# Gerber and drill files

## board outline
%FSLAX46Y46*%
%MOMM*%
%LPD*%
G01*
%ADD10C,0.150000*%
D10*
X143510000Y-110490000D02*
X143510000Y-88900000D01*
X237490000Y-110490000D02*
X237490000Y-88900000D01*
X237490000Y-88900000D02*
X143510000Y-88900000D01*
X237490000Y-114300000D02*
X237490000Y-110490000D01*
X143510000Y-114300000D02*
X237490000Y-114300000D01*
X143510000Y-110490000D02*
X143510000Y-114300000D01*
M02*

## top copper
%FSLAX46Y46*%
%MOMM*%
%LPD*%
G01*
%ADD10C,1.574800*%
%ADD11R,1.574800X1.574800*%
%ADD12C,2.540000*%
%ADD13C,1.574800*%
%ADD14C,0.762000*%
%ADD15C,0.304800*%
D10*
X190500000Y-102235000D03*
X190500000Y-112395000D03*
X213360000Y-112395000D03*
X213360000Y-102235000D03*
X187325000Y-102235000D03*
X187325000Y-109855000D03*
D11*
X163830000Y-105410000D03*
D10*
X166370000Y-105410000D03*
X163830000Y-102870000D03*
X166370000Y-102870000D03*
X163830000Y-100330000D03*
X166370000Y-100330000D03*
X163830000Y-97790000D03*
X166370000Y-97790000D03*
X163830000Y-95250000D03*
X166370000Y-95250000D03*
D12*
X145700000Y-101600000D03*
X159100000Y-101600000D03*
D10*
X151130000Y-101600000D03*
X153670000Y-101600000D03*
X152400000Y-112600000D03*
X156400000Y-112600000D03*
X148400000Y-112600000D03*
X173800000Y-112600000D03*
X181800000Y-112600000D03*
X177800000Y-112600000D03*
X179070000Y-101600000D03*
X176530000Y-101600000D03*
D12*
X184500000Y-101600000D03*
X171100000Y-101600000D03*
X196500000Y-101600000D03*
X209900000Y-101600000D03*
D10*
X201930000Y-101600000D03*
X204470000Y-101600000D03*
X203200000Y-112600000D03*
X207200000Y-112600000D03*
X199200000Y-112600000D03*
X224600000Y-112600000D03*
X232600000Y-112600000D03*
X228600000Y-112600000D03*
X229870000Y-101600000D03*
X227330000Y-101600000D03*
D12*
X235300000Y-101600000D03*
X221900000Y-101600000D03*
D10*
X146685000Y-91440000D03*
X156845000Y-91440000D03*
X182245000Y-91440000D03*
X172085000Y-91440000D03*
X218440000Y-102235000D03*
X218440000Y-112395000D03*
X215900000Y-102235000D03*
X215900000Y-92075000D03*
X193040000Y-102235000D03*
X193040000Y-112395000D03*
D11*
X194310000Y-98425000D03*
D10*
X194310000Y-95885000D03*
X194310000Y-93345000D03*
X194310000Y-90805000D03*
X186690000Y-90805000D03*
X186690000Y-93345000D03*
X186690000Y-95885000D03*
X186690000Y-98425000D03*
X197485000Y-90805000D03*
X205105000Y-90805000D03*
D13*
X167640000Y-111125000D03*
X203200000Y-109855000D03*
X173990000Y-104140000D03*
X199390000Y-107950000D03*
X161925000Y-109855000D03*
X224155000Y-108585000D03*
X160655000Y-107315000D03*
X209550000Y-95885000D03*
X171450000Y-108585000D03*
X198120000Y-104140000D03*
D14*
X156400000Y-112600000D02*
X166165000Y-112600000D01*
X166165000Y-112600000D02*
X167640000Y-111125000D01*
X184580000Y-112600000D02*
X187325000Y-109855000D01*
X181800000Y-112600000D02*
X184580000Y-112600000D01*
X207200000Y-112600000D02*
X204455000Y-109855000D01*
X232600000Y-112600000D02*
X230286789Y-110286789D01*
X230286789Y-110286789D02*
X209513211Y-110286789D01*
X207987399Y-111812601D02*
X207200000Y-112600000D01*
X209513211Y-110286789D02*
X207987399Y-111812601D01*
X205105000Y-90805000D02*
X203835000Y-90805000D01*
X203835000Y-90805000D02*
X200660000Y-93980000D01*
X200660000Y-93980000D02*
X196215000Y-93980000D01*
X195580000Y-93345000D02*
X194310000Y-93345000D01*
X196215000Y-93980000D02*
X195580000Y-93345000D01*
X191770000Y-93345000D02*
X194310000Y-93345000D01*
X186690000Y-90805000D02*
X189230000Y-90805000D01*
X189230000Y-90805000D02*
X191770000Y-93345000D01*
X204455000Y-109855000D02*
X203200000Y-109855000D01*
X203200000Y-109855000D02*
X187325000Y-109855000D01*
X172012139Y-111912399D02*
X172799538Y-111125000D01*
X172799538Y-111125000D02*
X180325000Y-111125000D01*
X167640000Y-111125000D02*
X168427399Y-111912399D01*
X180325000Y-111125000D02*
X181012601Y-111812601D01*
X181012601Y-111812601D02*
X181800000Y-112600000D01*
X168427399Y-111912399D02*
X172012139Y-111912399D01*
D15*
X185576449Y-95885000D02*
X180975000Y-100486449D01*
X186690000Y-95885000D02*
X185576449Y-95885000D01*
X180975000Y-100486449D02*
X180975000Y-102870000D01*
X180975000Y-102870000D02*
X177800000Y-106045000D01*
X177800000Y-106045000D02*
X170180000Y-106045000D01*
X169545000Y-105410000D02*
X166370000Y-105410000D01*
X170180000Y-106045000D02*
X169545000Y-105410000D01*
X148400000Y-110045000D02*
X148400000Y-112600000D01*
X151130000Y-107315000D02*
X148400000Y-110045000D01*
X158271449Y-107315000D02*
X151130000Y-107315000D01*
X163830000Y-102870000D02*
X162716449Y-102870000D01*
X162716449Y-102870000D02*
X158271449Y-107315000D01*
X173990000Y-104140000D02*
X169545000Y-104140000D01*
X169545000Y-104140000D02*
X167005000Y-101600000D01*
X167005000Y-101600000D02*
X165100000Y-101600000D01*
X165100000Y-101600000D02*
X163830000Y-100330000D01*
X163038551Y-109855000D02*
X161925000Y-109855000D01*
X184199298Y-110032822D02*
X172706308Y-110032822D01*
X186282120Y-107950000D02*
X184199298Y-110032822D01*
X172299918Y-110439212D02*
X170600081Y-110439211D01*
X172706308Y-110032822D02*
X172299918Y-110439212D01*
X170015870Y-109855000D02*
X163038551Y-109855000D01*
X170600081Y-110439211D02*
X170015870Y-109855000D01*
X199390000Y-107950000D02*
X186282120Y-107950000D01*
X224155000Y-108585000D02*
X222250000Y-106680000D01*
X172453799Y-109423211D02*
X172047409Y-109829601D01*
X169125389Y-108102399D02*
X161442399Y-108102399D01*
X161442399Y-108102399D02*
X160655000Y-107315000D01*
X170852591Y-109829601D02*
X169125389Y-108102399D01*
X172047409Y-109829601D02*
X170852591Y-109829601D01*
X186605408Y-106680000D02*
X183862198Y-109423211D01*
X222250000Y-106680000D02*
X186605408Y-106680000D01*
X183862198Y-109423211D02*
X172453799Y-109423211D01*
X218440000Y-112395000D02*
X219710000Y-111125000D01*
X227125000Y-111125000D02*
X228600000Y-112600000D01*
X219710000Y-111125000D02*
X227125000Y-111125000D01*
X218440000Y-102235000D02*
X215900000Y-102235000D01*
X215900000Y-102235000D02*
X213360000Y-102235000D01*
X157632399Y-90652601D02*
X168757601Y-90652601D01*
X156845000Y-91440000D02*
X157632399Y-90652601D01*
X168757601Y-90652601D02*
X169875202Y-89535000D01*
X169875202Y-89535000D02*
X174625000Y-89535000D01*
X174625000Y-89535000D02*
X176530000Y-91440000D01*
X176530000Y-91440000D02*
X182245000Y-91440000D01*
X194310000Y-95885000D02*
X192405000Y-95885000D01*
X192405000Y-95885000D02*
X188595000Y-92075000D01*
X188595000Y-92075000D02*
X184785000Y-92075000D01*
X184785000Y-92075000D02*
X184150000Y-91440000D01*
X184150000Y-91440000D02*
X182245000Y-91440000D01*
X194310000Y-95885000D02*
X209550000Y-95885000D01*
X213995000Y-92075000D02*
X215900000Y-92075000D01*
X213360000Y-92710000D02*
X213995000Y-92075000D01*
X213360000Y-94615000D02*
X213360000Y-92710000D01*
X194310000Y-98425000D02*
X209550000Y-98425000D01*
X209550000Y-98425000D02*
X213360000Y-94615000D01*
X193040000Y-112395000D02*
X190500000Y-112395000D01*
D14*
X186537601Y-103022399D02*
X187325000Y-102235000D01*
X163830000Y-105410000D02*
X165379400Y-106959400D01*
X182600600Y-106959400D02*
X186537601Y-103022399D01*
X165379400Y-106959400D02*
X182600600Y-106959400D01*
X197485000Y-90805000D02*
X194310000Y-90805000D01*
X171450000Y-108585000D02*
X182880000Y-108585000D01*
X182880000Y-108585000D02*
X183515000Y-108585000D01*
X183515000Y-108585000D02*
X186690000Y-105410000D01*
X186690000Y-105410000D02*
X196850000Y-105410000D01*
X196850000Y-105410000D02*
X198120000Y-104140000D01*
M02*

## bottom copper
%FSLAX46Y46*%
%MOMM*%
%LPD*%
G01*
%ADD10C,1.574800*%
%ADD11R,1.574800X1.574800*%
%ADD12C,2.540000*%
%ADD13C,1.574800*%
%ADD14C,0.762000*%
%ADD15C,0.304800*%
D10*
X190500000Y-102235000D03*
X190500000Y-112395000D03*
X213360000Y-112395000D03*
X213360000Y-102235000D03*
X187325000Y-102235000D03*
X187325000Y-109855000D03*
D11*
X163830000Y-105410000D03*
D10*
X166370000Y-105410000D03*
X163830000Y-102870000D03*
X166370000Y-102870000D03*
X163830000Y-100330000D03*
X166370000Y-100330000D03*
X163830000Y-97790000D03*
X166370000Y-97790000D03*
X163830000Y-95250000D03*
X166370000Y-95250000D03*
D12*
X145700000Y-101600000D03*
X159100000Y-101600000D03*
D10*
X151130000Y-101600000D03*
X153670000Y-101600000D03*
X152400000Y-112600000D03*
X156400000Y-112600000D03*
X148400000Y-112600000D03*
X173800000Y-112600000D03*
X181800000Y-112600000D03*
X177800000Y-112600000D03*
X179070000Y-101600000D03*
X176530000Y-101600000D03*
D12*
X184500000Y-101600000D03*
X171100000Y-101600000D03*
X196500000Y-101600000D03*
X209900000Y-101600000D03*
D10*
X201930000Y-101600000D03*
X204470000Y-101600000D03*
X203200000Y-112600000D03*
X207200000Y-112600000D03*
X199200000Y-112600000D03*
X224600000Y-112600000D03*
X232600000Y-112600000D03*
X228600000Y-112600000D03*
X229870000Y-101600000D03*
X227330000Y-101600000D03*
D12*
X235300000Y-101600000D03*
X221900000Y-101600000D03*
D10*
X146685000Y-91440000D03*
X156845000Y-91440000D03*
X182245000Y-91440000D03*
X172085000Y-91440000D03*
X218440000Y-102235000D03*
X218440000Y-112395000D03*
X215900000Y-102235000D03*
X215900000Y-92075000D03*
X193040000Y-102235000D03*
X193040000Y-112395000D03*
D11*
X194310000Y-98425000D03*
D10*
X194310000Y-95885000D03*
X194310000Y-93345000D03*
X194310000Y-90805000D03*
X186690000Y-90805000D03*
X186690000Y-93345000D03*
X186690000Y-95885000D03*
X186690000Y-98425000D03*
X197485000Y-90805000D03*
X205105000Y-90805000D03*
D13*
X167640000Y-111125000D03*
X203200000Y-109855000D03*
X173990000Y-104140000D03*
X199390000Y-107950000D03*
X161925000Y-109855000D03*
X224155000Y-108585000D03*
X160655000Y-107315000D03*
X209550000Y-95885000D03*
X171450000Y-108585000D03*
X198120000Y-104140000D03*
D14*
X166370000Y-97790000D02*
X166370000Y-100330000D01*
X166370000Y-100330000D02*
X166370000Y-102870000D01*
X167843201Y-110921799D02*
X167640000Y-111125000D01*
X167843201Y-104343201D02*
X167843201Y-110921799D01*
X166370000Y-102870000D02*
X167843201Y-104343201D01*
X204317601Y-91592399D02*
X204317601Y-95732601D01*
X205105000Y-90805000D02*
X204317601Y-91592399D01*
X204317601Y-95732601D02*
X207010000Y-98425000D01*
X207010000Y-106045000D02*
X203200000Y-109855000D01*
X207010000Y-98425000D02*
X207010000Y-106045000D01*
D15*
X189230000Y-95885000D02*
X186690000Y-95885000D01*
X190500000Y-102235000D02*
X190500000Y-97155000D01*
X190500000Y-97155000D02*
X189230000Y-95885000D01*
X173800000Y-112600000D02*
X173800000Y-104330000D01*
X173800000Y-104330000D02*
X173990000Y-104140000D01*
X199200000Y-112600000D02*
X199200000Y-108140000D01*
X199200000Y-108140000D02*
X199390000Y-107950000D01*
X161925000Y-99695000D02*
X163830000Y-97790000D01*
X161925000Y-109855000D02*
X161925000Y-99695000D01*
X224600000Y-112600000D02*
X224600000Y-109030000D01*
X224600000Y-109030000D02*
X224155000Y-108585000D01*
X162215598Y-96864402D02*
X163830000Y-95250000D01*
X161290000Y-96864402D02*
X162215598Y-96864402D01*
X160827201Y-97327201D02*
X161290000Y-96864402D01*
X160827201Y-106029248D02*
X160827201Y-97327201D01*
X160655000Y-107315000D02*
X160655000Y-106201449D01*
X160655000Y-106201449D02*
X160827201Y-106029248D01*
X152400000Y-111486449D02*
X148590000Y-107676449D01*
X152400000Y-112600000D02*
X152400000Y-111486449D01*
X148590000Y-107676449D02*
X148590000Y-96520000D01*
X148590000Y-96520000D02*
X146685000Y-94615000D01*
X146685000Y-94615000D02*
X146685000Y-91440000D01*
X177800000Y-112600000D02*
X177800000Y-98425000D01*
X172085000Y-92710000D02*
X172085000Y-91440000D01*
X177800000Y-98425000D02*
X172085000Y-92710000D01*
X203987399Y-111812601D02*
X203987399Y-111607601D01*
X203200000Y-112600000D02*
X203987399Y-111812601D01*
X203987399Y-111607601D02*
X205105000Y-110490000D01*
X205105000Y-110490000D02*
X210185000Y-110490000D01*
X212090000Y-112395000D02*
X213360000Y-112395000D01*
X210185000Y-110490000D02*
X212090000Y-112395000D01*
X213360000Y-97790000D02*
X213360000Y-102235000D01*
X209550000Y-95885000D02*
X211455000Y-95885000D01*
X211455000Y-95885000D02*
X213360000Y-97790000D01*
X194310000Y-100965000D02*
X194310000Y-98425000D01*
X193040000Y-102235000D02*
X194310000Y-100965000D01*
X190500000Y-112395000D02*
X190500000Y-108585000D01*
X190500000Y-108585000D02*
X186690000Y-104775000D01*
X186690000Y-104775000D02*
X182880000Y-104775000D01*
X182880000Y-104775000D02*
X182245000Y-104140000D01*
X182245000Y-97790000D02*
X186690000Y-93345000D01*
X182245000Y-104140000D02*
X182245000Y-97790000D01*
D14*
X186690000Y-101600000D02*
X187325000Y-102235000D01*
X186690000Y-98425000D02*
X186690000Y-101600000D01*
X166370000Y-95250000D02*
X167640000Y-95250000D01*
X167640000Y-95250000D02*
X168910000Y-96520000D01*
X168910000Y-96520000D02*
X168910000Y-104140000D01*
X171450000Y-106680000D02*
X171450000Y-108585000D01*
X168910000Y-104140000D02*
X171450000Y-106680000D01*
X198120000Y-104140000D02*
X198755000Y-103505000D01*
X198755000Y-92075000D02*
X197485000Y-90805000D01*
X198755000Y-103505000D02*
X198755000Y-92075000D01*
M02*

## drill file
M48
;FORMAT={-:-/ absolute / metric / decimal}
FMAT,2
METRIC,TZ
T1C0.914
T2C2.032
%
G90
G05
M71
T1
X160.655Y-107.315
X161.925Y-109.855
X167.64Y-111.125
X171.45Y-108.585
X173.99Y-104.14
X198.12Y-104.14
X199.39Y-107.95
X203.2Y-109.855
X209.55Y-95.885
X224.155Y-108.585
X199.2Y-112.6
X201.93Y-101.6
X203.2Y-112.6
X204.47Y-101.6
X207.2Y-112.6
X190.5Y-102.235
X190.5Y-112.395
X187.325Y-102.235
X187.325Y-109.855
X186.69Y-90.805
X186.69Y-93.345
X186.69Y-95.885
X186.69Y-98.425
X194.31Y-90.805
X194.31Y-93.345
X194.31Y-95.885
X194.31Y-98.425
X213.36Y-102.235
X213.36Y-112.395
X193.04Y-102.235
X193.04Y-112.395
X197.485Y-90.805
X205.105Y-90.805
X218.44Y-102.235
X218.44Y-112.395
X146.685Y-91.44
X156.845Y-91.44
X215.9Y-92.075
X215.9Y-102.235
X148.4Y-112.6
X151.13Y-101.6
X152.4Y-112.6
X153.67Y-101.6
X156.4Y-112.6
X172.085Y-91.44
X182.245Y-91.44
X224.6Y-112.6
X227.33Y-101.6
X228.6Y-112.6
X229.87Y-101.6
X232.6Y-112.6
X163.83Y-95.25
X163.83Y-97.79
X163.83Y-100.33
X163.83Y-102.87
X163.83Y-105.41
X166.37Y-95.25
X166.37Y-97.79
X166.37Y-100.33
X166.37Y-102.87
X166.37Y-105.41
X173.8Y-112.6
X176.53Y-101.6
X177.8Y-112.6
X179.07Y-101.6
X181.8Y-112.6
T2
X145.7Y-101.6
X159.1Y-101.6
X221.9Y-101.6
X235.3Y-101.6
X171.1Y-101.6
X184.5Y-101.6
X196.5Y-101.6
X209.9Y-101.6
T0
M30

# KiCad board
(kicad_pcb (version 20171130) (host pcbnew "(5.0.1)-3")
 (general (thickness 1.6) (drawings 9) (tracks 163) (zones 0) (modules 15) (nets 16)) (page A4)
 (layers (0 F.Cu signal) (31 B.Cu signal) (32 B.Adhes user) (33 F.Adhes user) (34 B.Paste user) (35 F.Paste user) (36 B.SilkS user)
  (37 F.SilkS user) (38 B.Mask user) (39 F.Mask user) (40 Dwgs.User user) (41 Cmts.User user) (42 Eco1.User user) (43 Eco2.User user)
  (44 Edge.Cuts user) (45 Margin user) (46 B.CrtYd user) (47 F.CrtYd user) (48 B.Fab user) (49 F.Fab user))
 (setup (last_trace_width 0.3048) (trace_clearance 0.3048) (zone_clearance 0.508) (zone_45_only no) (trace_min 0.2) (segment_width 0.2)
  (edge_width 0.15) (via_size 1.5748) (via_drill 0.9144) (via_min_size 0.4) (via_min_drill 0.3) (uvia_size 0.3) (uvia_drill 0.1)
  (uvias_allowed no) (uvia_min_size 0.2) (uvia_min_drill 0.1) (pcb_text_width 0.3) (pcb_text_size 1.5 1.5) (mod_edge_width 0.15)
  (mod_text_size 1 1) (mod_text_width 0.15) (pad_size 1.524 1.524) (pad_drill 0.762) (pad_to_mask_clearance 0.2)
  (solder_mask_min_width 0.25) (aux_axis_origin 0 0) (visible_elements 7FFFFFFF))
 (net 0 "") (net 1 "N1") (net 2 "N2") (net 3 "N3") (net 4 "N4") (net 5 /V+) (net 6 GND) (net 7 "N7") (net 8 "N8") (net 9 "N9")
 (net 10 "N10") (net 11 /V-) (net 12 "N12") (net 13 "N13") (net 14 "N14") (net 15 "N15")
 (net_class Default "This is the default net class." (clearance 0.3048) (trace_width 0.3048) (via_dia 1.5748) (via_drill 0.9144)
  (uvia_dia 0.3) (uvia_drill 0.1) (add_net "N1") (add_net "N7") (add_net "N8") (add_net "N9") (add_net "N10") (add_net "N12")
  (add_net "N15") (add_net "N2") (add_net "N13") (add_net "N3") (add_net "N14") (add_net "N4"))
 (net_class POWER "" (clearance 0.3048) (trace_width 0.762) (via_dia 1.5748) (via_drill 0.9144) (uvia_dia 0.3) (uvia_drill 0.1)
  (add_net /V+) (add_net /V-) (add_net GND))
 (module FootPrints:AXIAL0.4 (layer F.Cu) (at 190.5 107.315 90)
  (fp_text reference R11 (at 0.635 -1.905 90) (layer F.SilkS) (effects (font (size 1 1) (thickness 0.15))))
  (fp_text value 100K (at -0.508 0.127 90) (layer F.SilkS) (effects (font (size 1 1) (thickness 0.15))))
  (pad 2 thru_hole circle (at 5.08 0 90) (size 1.5748 1.5748) (drill 0.9144) (layers *.Cu *.Mask F.SilkS) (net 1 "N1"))
  (pad 1 thru_hole circle (at -5.08 0 90) (size 1.5748 1.5748) (drill 0.9144) (layers *.Cu *.Mask F.SilkS) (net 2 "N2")))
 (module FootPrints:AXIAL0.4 (layer F.Cu) (at 213.36 107.315 90)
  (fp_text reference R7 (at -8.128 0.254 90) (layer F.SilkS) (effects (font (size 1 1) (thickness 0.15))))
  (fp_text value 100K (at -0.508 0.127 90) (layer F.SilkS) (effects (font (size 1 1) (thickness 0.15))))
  (pad 1 thru_hole circle (at -5.08 0 90) (size 1.5748 1.5748) (drill 0.9144) (layers *.Cu *.Mask F.SilkS) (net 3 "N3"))
  (pad 2 thru_hole circle (at 5.08 0 90) (size 1.5748 1.5748) (drill 0.9144) (layers *.Cu *.Mask F.SilkS) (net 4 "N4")))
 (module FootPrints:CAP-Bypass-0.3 (layer F.Cu) (at 187.325 106.045 270)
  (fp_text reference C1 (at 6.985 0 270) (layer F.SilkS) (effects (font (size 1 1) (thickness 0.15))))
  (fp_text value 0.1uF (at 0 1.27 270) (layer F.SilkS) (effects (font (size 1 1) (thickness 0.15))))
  (pad 1 thru_hole circle (at -3.81 0 270) (size 1.5748 1.5748) (drill 0.9144) (layers *.Cu *.Mask F.SilkS) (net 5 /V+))
  (pad 2 thru_hole circle (at 3.81 0 270) (size 1.5748 1.5748) (drill 0.9144) (layers *.Cu *.Mask F.SilkS) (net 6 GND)))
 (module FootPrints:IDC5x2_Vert (layer B.Cu) (at 165.1 100.33 270)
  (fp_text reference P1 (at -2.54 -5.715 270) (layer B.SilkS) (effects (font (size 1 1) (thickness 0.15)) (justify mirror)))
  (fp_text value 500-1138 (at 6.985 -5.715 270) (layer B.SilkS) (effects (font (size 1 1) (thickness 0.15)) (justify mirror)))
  (pad 1 thru_hole rect (at 5.08 1.27 270) (size 1.5748 1.5748) (drill 0.9144) (layers *.Cu *.Mask B.SilkS) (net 5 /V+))
  (pad 2 thru_hole circle (at 5.08 -1.27 270) (size 1.5748 1.5748) (drill 0.9144) (layers *.Cu *.Mask B.SilkS) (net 1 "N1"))
  (pad 3 thru_hole circle (at 2.54 1.27 270) (size 1.5748 1.5748) (drill 0.9144) (layers *.Cu *.Mask B.SilkS) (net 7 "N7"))
  (pad 4 thru_hole circle (at 2.54 -1.27 270) (size 1.5748 1.5748) (drill 0.9144) (layers *.Cu *.Mask B.SilkS) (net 6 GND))
  (pad 5 thru_hole circle (at 0 1.27 270) (size 1.5748 1.5748) (drill 0.9144) (layers *.Cu *.Mask B.SilkS) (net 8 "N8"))
  (pad 6 thru_hole circle (at 0 -1.27 270) (size 1.5748 1.5748) (drill 0.9144) (layers *.Cu *.Mask B.SilkS) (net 6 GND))
  (pad 7 thru_hole circle (at -2.54 1.27 270) (size 1.5748 1.5748) (drill 0.9144) (layers *.Cu *.Mask B.SilkS) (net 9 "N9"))
  (pad 8 thru_hole circle (at -2.54 -1.27 270) (size 1.5748 1.5748) (drill 0.9144) (layers *.Cu *.Mask B.SilkS) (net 6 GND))
  (pad 9 thru_hole circle (at -5.08 1.27 270) (size 1.5748 1.5748) (drill 0.9144) (layers *.Cu *.Mask B.SilkS) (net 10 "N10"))
  (pad 10 thru_hole circle (at -5.08 -1.27 270) (size 1.5748 1.5748) (drill 0.9144) (layers *.Cu *.Mask B.SilkS) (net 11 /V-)))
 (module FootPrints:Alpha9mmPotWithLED (layer F.Cu) (at 152.4 101.6)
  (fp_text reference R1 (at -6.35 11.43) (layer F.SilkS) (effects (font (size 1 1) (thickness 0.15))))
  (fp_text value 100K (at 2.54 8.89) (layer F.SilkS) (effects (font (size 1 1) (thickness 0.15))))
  (pad "" thru_hole circle (at -6.7 0) (size 2.54 2.54) (drill 2.032) (layers *.Cu *.Mask F.SilkS))
  (pad "" thru_hole circle (at 6.7 0) (size 2.54 2.54) (drill 2.032) (layers *.Cu *.Mask F.SilkS))
  (pad 4 thru_hole circle (at -1.27 0) (size 1.5748 1.5748) (drill 0.9144) (layers *.Cu *.Mask F.SilkS))
  (pad 5 thru_hole circle (at 1.27 0) (size 1.5748 1.5748) (drill 0.9144) (layers *.Cu *.Mask F.SilkS))
  (pad 2 thru_hole circle (at 0 11) (size 1.5748 1.5748) (drill 0.9144) (layers *.Cu *.Mask F.SilkS) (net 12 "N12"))
  (pad 3 thru_hole circle (at 4 11) (size 1.5748 1.5748) (drill 0.9144) (layers *.Cu *.Mask F.SilkS) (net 6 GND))
  (pad 1 thru_hole circle (at -4 11) (size 1.5748 1.5748) (drill 0.9144) (layers *.Cu *.Mask F.SilkS) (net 7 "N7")))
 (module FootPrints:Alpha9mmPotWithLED (layer F.Cu) (at 177.8 101.6)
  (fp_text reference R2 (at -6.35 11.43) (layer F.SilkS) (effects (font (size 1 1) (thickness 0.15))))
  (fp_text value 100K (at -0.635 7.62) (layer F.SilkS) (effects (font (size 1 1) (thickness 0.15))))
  (pad 1 thru_hole circle (at -4 11) (size 1.5748 1.5748) (drill 0.9144) (layers *.Cu *.Mask F.SilkS) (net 8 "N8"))
  (pad 3 thru_hole circle (at 4 11) (size 1.5748 1.5748) (drill 0.9144) (layers *.Cu *.Mask F.SilkS) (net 6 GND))
  (pad 2 thru_hole circle (at 0 11) (size 1.5748 1.5748) (drill 0.9144) (layers *.Cu *.Mask F.SilkS) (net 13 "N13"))
  (pad 5 thru_hole circle (at 1.27 0) (size 1.5748 1.5748) (drill 0.9144) (layers *.Cu *.Mask F.SilkS))
  (pad 4 thru_hole circle (at -1.27 0) (size 1.5748 1.5748) (drill 0.9144) (layers *.Cu *.Mask F.SilkS))
  (pad "" thru_hole circle (at 6.7 0) (size 2.54 2.54) (drill 2.032) (layers *.Cu *.Mask F.SilkS))
  (pad "" thru_hole circle (at -6.7 0) (size 2.54 2.54) (drill 2.032) (layers *.Cu *.Mask F.SilkS)))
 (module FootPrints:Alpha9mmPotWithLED (layer F.Cu) (at 203.2 101.6)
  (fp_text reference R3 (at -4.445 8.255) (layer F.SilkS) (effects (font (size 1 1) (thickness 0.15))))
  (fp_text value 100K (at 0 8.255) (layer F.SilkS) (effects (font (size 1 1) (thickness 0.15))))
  (pad "" thru_hole circle (at -6.7 0) (size 2.54 2.54) (drill 2.032) (layers *.Cu *.Mask F.SilkS))
  (pad "" thru_hole circle (at 6.7 0) (size 2.54 2.54) (drill 2.032) (layers *.Cu *.Mask F.SilkS))
  (pad 4 thru_hole circle (at -1.27 0) (size 1.5748 1.5748) (drill 0.9144) (layers *.Cu *.Mask F.SilkS))
  (pad 5 thru_hole circle (at 1.27 0) (size 1.5748 1.5748) (drill 0.9144) (layers *.Cu *.Mask F.SilkS))
  (pad 2 thru_hole circle (at 0 11) (size 1.5748 1.5748) (drill 0.9144) (layers *.Cu *.Mask F.SilkS) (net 3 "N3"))
  (pad 3 thru_hole circle (at 4 11) (size 1.5748 1.5748) (drill 0.9144) (layers *.Cu *.Mask F.SilkS) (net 6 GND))
  (pad 1 thru_hole circle (at -4 11) (size 1.5748 1.5748) (drill 0.9144) (layers *.Cu *.Mask F.SilkS) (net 9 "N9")))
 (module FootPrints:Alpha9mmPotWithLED (layer F.Cu) (at 228.6 101.6)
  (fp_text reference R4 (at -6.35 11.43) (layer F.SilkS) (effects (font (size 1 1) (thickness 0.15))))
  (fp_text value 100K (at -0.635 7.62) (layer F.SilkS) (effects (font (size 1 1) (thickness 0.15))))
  (pad 1 thru_hole circle (at -4 11) (size 1.5748 1.5748) (drill 0.9144) (layers *.Cu *.Mask F.SilkS) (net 10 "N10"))
  (pad 3 thru_hole circle (at 4 11) (size 1.5748 1.5748) (drill 0.9144) (layers *.Cu *.Mask F.SilkS) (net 6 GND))
  (pad 2 thru_hole circle (at 0 11) (size 1.5748 1.5748) (drill 0.9144) (layers *.Cu *.Mask F.SilkS) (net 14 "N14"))
  (pad 5 thru_hole circle (at 1.27 0) (size 1.5748 1.5748) (drill 0.9144) (layers *.Cu *.Mask F.SilkS))
  (pad 4 thru_hole circle (at -1.27 0) (size 1.5748 1.5748) (drill 0.9144) (layers *.Cu *.Mask F.SilkS))
  (pad "" thru_hole circle (at 6.7 0) (size 2.54 2.54) (drill 2.032) (layers *.Cu *.Mask F.SilkS))
  (pad "" thru_hole circle (at -6.7 0) (size 2.54 2.54) (drill 2.032) (layers *.Cu *.Mask F.SilkS)))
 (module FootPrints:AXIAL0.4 (layer F.Cu) (at 151.765 91.44)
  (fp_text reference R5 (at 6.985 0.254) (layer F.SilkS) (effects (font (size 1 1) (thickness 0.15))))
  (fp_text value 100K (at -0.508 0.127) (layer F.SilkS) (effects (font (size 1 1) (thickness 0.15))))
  (pad 1 thru_hole circle (at -5.08 0) (size 1.5748 1.5748) (drill 0.9144) (layers *.Cu *.Mask F.SilkS) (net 12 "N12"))
  (pad 2 thru_hole circle (at 5.08 0) (size 1.5748 1.5748) (drill 0.9144) (layers *.Cu *.Mask F.SilkS) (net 4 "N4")))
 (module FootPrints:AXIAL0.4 (layer F.Cu) (at 177.165 91.44)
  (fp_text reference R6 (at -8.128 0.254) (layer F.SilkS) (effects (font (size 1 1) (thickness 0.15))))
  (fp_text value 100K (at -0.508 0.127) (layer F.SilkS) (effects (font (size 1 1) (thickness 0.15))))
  (pad 2 thru_hole circle (at 5.08 0) (size 1.5748 1.5748) (drill 0.9144) (layers *.Cu *.Mask F.SilkS) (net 4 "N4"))
  (pad 1 thru_hole circle (at -5.08 0) (size 1.5748 1.5748) (drill 0.9144) (layers *.Cu *.Mask F.SilkS) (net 13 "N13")))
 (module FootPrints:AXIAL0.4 (layer F.Cu) (at 218.44 107.315 90)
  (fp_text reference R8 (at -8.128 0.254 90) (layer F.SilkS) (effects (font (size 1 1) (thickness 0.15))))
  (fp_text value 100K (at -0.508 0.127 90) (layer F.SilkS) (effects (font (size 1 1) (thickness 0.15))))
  (pad 2 thru_hole circle (at 5.08 0 90) (size 1.5748 1.5748) (drill 0.9144) (layers *.Cu *.Mask F.SilkS) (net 4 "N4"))
  (pad 1 thru_hole circle (at -5.08 0 90) (size 1.5748 1.5748) (drill 0.9144) (layers *.Cu *.Mask F.SilkS) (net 14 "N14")))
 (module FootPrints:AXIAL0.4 (layer F.Cu) (at 215.9 97.155 90)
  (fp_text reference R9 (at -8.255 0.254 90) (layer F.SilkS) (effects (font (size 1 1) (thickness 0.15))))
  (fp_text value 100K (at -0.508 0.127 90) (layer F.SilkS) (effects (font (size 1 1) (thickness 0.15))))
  (pad 1 thru_hole circle (at -5.08 0 90) (size 1.5748 1.5748) (drill 0.9144) (layers *.Cu *.Mask F.SilkS) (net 4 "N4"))
  (pad 2 thru_hole circle (at 5.08 0 90) (size 1.5748 1.5748) (drill 0.9144) (layers *.Cu *.Mask F.SilkS) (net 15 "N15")))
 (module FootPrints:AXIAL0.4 (layer F.Cu) (at 193.04 107.315 270)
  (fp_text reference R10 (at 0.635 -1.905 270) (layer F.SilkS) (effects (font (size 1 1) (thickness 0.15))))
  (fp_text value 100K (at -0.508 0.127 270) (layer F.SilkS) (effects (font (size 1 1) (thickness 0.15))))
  (pad 1 thru_hole circle (at -5.08 0 270) (size 1.5748 1.5748) (drill 0.9144) (layers *.Cu *.Mask F.SilkS) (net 15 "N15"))
  (pad 2 thru_hole circle (at 5.08 0 270) (size 1.5748 1.5748) (drill 0.9144) (layers *.Cu *.Mask F.SilkS) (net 2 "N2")))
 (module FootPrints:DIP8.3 (layer F.Cu) (at 190.5 94.615 90)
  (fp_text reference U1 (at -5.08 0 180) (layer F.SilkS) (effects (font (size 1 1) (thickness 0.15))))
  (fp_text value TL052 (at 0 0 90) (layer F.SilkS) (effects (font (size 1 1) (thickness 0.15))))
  (pad 1 thru_hole rect (at -3.81 3.81 90) (size 1.5748 1.5748) (drill 0.9144) (layers *.Cu *.Mask F.SilkS) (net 15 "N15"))
  (pad 2 thru_hole circle (at -1.27 3.81 90) (size 1.5748 1.5748) (drill 0.9144) (layers *.Cu *.Mask F.SilkS) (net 4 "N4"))
  (pad 3 thru_hole circle (at 1.27 3.81 90) (size 1.5748 1.5748) (drill 0.9144) (layers *.Cu *.Mask F.SilkS) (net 6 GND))
  (pad 4 thru_hole circle (at 3.81 3.81 90) (size 1.5748 1.5748) (drill 0.9144) (layers *.Cu *.Mask F.SilkS) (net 11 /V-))
  (pad 5 thru_hole circle (at 3.81 -3.81 90) (size 1.5748 1.5748) (drill 0.9144) (layers *.Cu *.Mask F.SilkS) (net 6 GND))
  (pad 6 thru_hole circle (at 1.27 -3.81 90) (size 1.5748 1.5748) (drill 0.9144) (layers *.Cu *.Mask F.SilkS) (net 2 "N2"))
  (pad 7 thru_hole circle (at -1.27 -3.81 90) (size 1.5748 1.5748) (drill 0.9144) (layers *.Cu *.Mask F.SilkS) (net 1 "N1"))
  (pad 8 thru_hole circle (at -3.81 -3.81 90) (size 1.5748 1.5748) (drill 0.9144) (layers *.Cu *.Mask F.SilkS) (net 5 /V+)))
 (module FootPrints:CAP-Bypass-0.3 (layer F.Cu) (at 201.295 90.805)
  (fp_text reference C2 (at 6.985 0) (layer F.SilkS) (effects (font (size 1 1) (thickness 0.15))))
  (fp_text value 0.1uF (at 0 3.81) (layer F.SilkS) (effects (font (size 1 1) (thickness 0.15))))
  (pad 1 thru_hole circle (at -3.81 0) (size 1.5748 1.5748) (drill 0.9144) (layers *.Cu *.Mask F.SilkS) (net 11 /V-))
  (pad 2 thru_hole circle (at 3.81 0) (size 1.5748 1.5748) (drill 0.9144) (layers *.Cu *.Mask F.SilkS) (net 6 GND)))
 (gr_line (start 143.51 110.49) (end 143.51 88.9) (layer Edge.Cuts) (width 0.15))
 (gr_line (start 237.49 110.49) (end 237.49 88.9) (layer Edge.Cuts) (width 0.15))
 (gr_line (start 237.49 88.9) (end 143.51 88.9) (layer Edge.Cuts) (width 0.15))
 (gr_line (start 237.49 114.3) (end 237.49 110.49) (layer Edge.Cuts) (width 0.15))
 (gr_line (start 143.51 114.3) (end 237.49 114.3) (layer Edge.Cuts) (width 0.15))
 (gr_line (start 143.51 110.49) (end 143.51 114.3) (layer Edge.Cuts) (width 0.15))
 (segment (start 156.4 112.6) (end 166.165 112.6) (width 0.762) (layer F.Cu) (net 6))
 (segment (start 166.165 112.6) (end 167.64 111.125) (width 0.762) (layer F.Cu) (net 6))
 (segment (start 184.58 112.6) (end 187.325 109.855) (width 0.762) (layer F.Cu) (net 6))
 (segment (start 181.8 112.6) (end 184.58 112.6) (width 0.762) (layer F.Cu) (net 6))
 (segment (start 207.2 112.6) (end 204.455 109.855) (width 0.762) (layer F.Cu) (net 6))
 (segment (start 232.6 112.6) (end 230.286789 110.286789) (width 0.762) (layer F.Cu) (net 6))
 (segment (start 230.286789 110.286789) (end 209.513211 110.286789) (width 0.762) (layer F.Cu) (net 6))
 (segment (start 207.987399 111.812601) (end 207.2 112.6) (width 0.762) (layer F.Cu) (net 6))
 (segment (start 209.513211 110.286789) (end 207.987399 111.812601) (width 0.762) (layer F.Cu) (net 6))
 (segment (start 166.37 97.79) (end 166.37 100.33) (width 0.762) (layer B.Cu) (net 6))
 (segment (start 166.37 100.33) (end 166.37 102.87) (width 0.762) (layer B.Cu) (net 6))
 (via (at 167.64 111.125) (size 1.5748) (drill 0.9144) (layers F.Cu B.Cu) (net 6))
 (segment (start 167.843201 110.921799) (end 167.64 111.125) (width 0.762) (layer B.Cu) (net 6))
 (segment (start 167.843201 104.343201) (end 167.843201 110.921799) (width 0.762) (layer B.Cu) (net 6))
 (segment (start 166.37 102.87) (end 167.843201 104.343201) (width 0.762) (layer B.Cu) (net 6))
 (segment (start 205.105 90.805) (end 203.835 90.805) (width 0.762) (layer F.Cu) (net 6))
 (segment (start 203.835 90.805) (end 200.66 93.98) (width 0.762) (layer F.Cu) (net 6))
 (segment (start 200.66 93.98) (end 196.215 93.98) (width 0.762) (layer F.Cu) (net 6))
 (segment (start 195.58 93.345) (end 194.31 93.345) (width 0.762) (layer F.Cu) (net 6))
 (segment (start 196.215 93.98) (end 195.58 93.345) (width 0.762) (layer F.Cu) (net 6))
 (segment (start 191.77 93.345) (end 194.31 93.345) (width 0.762) (layer F.Cu) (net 6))
 (segment (start 186.69 90.805) (end 189.23 90.805) (width 0.762) (layer F.Cu) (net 6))
 (segment (start 189.23 90.805) (end 191.77 93.345) (width 0.762) (layer F.Cu) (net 6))
 (segment (start 204.317601 91.592399) (end 204.317601 95.732601) (width 0.762) (layer B.Cu) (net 6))
 (segment (start 205.105 90.805) (end 204.317601 91.592399) (width 0.762) (layer B.Cu) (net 6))
 (segment (start 204.317601 95.732601) (end 207.01 98.425) (width 0.762) (layer B.Cu) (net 6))
 (via (at 203.2 109.855) (size 1.5748) (drill 0.9144) (layers F.Cu B.Cu) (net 6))
 (segment (start 207.01 106.045) (end 203.2 109.855) (width 0.762) (layer B.Cu) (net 6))
 (segment (start 207.01 98.425) (end 207.01 106.045) (width 0.762) (layer B.Cu) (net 6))
 (segment (start 204.455 109.855) (end 203.2 109.855) (width 0.762) (layer F.Cu) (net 6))
 (segment (start 203.2 109.855) (end 187.325 109.855) (width 0.762) (layer F.Cu) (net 6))
 (segment (start 172.012139 111.912399) (end 172.799538 111.125) (width 0.762) (layer F.Cu) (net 6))
 (segment (start 172.799538 111.125) (end 180.325 111.125) (width 0.762) (layer F.Cu) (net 6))
 (segment (start 167.64 111.125) (end 168.427399 111.912399) (width 0.762) (layer F.Cu) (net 6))
 (segment (start 180.325 111.125) (end 181.012601 111.812601) (width 0.762) (layer F.Cu) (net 6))
 (segment (start 181.012601 111.812601) (end 181.8 112.6) (width 0.762) (layer F.Cu) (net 6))
 (segment (start 168.427399 111.912399) (end 172.012139 111.912399) (width 0.762) (layer F.Cu) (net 6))
 (segment (start 189.23 95.885) (end 186.69 95.885) (width 0.3048) (layer B.Cu) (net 1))
 (segment (start 190.5 102.235) (end 190.5 97.155) (width 0.3048) (layer B.Cu) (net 1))
 (segment (start 190.5 97.155) (end 189.23 95.885) (width 0.3048) (layer B.Cu) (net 1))
 (segment (start 185.576449 95.885) (end 180.975 100.486449) (width 0.3048) (layer F.Cu) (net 1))
 (segment (start 186.69 95.885) (end 185.576449 95.885) (width 0.3048) (layer F.Cu) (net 1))
 (segment (start 180.975 100.486449) (end 180.975 102.87) (width 0.3048) (layer F.Cu) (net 1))
 (segment (start 180.975 102.87) (end 177.8 106.045) (width 0.3048) (layer F.Cu) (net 1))
 (segment (start 177.8 106.045) (end 170.18 106.045) (width 0.3048) (layer F.Cu) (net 1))
 (segment (start 169.545 105.41) (end 166.37 105.41) (width 0.3048) (layer F.Cu) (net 1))
 (segment (start 170.18 106.045) (end 169.545 105.41) (width 0.3048) (layer F.Cu) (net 1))
 (segment (start 148.4 110.045) (end 148.4 112.6) (width 0.3048) (layer F.Cu) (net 7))
 (segment (start 151.13 107.315) (end 148.4 110.045) (width 0.3048) (layer F.Cu) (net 7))
 (segment (start 158.271449 107.315) (end 151.13 107.315) (width 0.3048) (layer F.Cu) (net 7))
 (segment (start 163.83 102.87) (end 162.716449 102.87) (width 0.3048) (layer F.Cu) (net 7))
 (segment (start 162.716449 102.87) (end 158.271449 107.315) (width 0.3048) (layer F.Cu) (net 7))
 (via (at 173.99 104.14) (size 1.5748) (drill 0.9144) (layers F.Cu B.Cu) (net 8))
 (segment (start 173.8 112.6) (end 173.8 104.33) (width 0.3048) (layer B.Cu) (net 8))
 (segment (start 173.8 104.33) (end 173.99 104.14) (width 0.3048) (layer B.Cu) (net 8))
 (segment (start 173.99 104.14) (end 169.545 104.14) (width 0.3048) (layer F.Cu) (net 8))
 (segment (start 169.545 104.14) (end 167.005 101.6) (width 0.3048) (layer F.Cu) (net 8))
 (segment (start 167.005 101.6) (end 165.1 101.6) (width 0.3048) (layer F.Cu) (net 8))
 (segment (start 165.1 101.6) (end 163.83 100.33) (width 0.3048) (layer F.Cu) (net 8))
 (via (at 199.39 107.95) (size 1.5748) (drill 0.9144) (layers F.Cu B.Cu) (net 9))
 (segment (start 199.2 112.6) (end 199.2 108.14) (width 0.3048) (layer B.Cu) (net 9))
 (segment (start 199.2 108.14) (end 199.39 107.95) (width 0.3048) (layer B.Cu) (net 9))
 (via (at 161.925 109.855) (size 1.5748) (drill 0.9144) (layers F.Cu B.Cu) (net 9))
 (segment (start 161.925 99.695) (end 163.83 97.79) (width 0.3048) (layer B.Cu) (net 9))
 (segment (start 161.925 109.855) (end 161.925 99.695) (width 0.3048) (layer B.Cu) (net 9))
 (segment (start 163.038551 109.855) (end 161.925 109.855) (width 0.3048) (layer F.Cu) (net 9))
 (segment (start 184.199298 110.032822) (end 172.706308 110.032822) (width 0.3048) (layer F.Cu) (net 9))
 (segment (start 186.28212 107.95) (end 184.199298 110.032822) (width 0.3048) (layer F.Cu) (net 9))
 (segment (start 172.299918 110.439212) (end 170.600081 110.439211) (width 0.3048) (layer F.Cu) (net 9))
 (segment (start 172.706308 110.032822) (end 172.299918 110.439212) (width 0.3048) (layer F.Cu) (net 9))
 (segment (start 170.01587 109.855) (end 163.038551 109.855) (width 0.3048) (layer F.Cu) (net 9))
 (segment (start 170.600081 110.439211) (end 170.01587 109.855) (width 0.3048) (layer F.Cu) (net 9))
 (segment (start 199.39 107.95) (end 186.28212 107.95) (width 0.3048) (layer F.Cu) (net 9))
 (via (at 224.155 108.585) (size 1.5748) (drill 0.9144) (layers F.Cu B.Cu) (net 10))
 (segment (start 224.6 112.6) (end 224.6 109.03) (width 0.3048) (layer B.Cu) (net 10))
 (segment (start 224.6 109.03) (end 224.155 108.585) (width 0.3048) (layer B.Cu) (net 10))
 (via (at 160.655 107.315) (size 1.5748) (drill 0.9144) (layers F.Cu B.Cu) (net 10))
 (segment (start 162.215598 96.864402) (end 163.83 95.25) (width 0.3048) (layer B.Cu) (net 10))
 (segment (start 161.29 96.864402) (end 162.215598 96.864402) (width 0.3048) (layer B.Cu) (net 10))
 (segment (start 160.827201 97.327201) (end 161.29 96.864402) (width 0.3048) (layer B.Cu) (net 10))
 (segment (start 160.827201 106.029248) (end 160.827201 97.327201) (width 0.3048) (layer B.Cu) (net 10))
 (segment (start 160.655 107.315) (end 160.655 106.201449) (width 0.3048) (layer B.Cu) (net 10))
 (segment (start 160.655 106.201449) (end 160.827201 106.029248) (width 0.3048) (layer B.Cu) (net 10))
 (segment (start 224.155 108.585) (end 222.25 106.68) (width 0.3048) (layer F.Cu) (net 10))
 (segment (start 172.453799 109.423211) (end 172.047409 109.829601) (width 0.3048) (layer F.Cu) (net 10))
 (segment (start 169.125389 108.102399) (end 161.442399 108.102399) (width 0.3048) (layer F.Cu) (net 10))
 (segment (start 161.442399 108.102399) (end 160.655 107.315) (width 0.3048) (layer F.Cu) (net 10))
 (segment (start 170.852591 109.829601) (end 169.125389 108.102399) (width 0.3048) (layer F.Cu) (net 10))
 (segment (start 172.047409 109.829601) (end 170.852591 109.829601) (width 0.3048) (layer F.Cu) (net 10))
 (segment (start 186.605408 106.68) (end 183.862198 109.423211) (width 0.3048) (layer F.Cu) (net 10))
 (segment (start 222.25 106.68) (end 186.605408 106.68) (width 0.3048) (layer F.Cu) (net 10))
 (segment (start 183.862198 109.423211) (end 172.453799 109.423211) (width 0.3048) (layer F.Cu) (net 10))
 (segment (start 152.4 111.486449) (end 148.59 107.676449) (width 0.3048) (layer B.Cu) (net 12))
 (segment (start 152.4 112.6) (end 152.4 111.486449) (width 0.3048) (layer B.Cu) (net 12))
 (segment (start 148.59 107.676449) (end 148.59 96.52) (width 0.3048) (layer B.Cu) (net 12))
 (segment (start 148.59 96.52) (end 146.685 94.615) (width 0.3048) (layer B.Cu) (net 12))
 (segment (start 146.685 94.615) (end 146.685 91.44) (width 0.3048) (layer B.Cu) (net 12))
 (segment (start 177.8 112.6) (end 177.8 98.425) (width 0.3048) (layer B.Cu) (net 13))
 (segment (start 172.085 92.71) (end 172.085 91.44) (width 0.3048) (layer B.Cu) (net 13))
 (segment (start 177.8 98.425) (end 172.085 92.71) (width 0.3048) (layer B.Cu) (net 13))
 (segment (start 203.987399 111.812601) (end 203.987399 111.607601) (width 0.3048) (layer B.Cu) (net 3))
 (segment (start 203.2 112.6) (end 203.987399 111.812601) (width 0.3048) (layer B.Cu) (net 3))
 (segment (start 203.987399 111.607601) (end 205.105 110.49) (width 0.3048) (layer B.Cu) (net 3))
 (segment (start 205.105 110.49) (end 210.185 110.49) (width 0.3048) (layer B.Cu) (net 3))
 (segment (start 212.09 112.395) (end 213.36 112.395) (width 0.3048) (layer B.Cu) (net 3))
 (segment (start 210.185 110.49) (end 212.09 112.395) (width 0.3048) (layer B.Cu) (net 3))
 (segment (start 218.44 112.395) (end 219.71 111.125) (width 0.3048) (layer F.Cu) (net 14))
 (segment (start 227.125 111.125) (end 228.6 112.6) (width 0.3048) (layer F.Cu) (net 14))
 (segment (start 219.71 111.125) (end 227.125 111.125) (width 0.3048) (layer F.Cu) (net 14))
 (segment (start 218.44 102.235) (end 215.9 102.235) (width 0.3048) (layer F.Cu) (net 4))
 (segment (start 215.9 102.235) (end 213.36 102.235) (width 0.3048) (layer F.Cu) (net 4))
 (segment (start 157.632399 90.652601) (end 168.757601 90.652601) (width 0.3048) (layer F.Cu) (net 4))
 (segment (start 156.845 91.44) (end 157.632399 90.652601) (width 0.3048) (layer F.Cu) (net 4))
 (segment (start 168.757601 90.652601) (end 169.875202 89.535) (width 0.3048) (layer F.Cu) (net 4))
 (segment (start 169.875202 89.535) (end 174.625 89.535) (width 0.3048) (layer F.Cu) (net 4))
 (segment (start 174.625 89.535) (end 176.53 91.44) (width 0.3048) (layer F.Cu) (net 4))
 (segment (start 176.53 91.44) (end 182.245 91.44) (width 0.3048) (layer F.Cu) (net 4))
 (segment (start 194.31 95.885) (end 192.405 95.885) (width 0.3048) (layer F.Cu) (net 4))
 (segment (start 192.405 95.885) (end 188.595 92.075) (width 0.3048) (layer F.Cu) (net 4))
 (segment (start 188.595 92.075) (end 184.785 92.075) (width 0.3048) (layer F.Cu) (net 4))
 (segment (start 184.785 92.075) (end 184.15 91.44) (width 0.3048) (layer F.Cu) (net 4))
 (segment (start 184.15 91.44) (end 182.245 91.44) (width 0.3048) (layer F.Cu) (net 4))
 (via (at 209.55 95.885) (size 1.5748) (drill 0.9144) (layers F.Cu B.Cu) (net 4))
 (segment (start 194.31 95.885) (end 209.55 95.885) (width 0.3048) (layer F.Cu) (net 4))
 (segment (start 213.36 97.79) (end 213.36 102.235) (width 0.3048) (layer B.Cu) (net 4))
 (segment (start 209.55 95.885) (end 211.455 95.885) (width 0.3048) (layer B.Cu) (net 4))
 (segment (start 211.455 95.885) (end 213.36 97.79) (width 0.3048) (layer B.Cu) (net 4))
 (segment (start 194.31 100.965) (end 194.31 98.425) (width 0.3048) (layer B.Cu) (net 15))
 (segment (start 193.04 102.235) (end 194.31 100.965) (width 0.3048) (layer B.Cu) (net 15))
 (segment (start 213.995 92.075) (end 215.9 92.075) (width 0.3048) (layer F.Cu) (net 15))
 (segment (start 213.36 92.71) (end 213.995 92.075) (width 0.3048) (layer F.Cu) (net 15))
 (segment (start 213.36 94.615) (end 213.36 92.71) (width 0.3048) (layer F.Cu) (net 15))
 (segment (start 194.31 98.425) (end 209.55 98.425) (width 0.3048) (layer F.Cu) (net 15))
 (segment (start 209.55 98.425) (end 213.36 94.615) (width 0.3048) (layer F.Cu) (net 15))
 (segment (start 193.04 112.395) (end 190.5 112.395) (width 0.3048) (layer F.Cu) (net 2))
 (segment (start 190.5 112.395) (end 190.5 108.585) (width 0.3048) (layer B.Cu) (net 2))
 (segment (start 190.5 108.585) (end 186.69 104.775) (width 0.3048) (layer B.Cu) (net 2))
 (segment (start 186.69 104.775) (end 182.88 104.775) (width 0.3048) (layer B.Cu) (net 2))
 (segment (start 182.88 104.775) (end 182.245 104.14) (width 0.3048) (layer B.Cu) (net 2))
 (segment (start 182.245 97.79) (end 186.69 93.345) (width 0.3048) (layer B.Cu) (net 2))
 (segment (start 182.245 104.14) (end 182.245 97.79) (width 0.3048) (layer B.Cu) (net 2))
 (segment (start 186.69 101.6) (end 187.325 102.235) (width 0.762) (layer B.Cu) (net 5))
 (segment (start 186.69 98.425) (end 186.69 101.6) (width 0.762) (layer B.Cu) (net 5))
 (segment (start 186.537601 103.022399) (end 187.325 102.235) (width 0.762) (layer F.Cu) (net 5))
 (segment (start 163.83 105.41) (end 165.3794 106.9594) (width 0.762) (layer F.Cu) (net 5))
 (segment (start 182.6006 106.9594) (end 186.537601 103.022399) (width 0.762) (layer F.Cu) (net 5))
 (segment (start 165.3794 106.9594) (end 182.6006 106.9594) (width 0.762) (layer F.Cu) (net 5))
 (segment (start 197.485 90.805) (end 194.31 90.805) (width 0.762) (layer F.Cu) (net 11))
 (segment (start 166.37 95.25) (end 167.64 95.25) (width 0.762) (layer B.Cu) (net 11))
 (segment (start 167.64 95.25) (end 168.91 96.52) (width 0.762) (layer B.Cu) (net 11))
 (segment (start 168.91 96.52) (end 168.91 104.14) (width 0.762) (layer B.Cu) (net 11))
 (segment (start 171.45 106.68) (end 171.45 108.585) (width 0.762) (layer B.Cu) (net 11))
 (segment (start 168.91 104.14) (end 171.45 106.68) (width 0.762) (layer B.Cu) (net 11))
 (via (at 171.45 108.585) (size 1.5748) (drill 0.9144) (layers F.Cu B.Cu) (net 11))
 (segment (start 171.45 108.585) (end 182.88 108.585) (width 0.762) (layer F.Cu) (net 11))
 (segment (start 182.88 108.585) (end 183.515 108.585) (width 0.762) (layer F.Cu) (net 11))
 (segment (start 183.515 108.585) (end 186.69 105.41) (width 0.762) (layer F.Cu) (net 11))
 (via (at 198.12 104.14) (size 1.5748) (drill 0.9144) (layers F.Cu B.Cu) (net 11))
 (segment (start 186.69 105.41) (end 196.85 105.41) (width 0.762) (layer F.Cu) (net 11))
 (segment (start 196.85 105.41) (end 198.12 104.14) (width 0.762) (layer F.Cu) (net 11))
 (segment (start 198.12 104.14) (end 198.755 103.505) (width 0.762) (layer B.Cu) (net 11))
 (segment (start 198.755 92.075) (end 197.485 90.805) (width 0.762) (layer B.Cu) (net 11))
 (segment (start 198.755 103.505) (end 198.755 92.075) (width 0.762) (layer B.Cu) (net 11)))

